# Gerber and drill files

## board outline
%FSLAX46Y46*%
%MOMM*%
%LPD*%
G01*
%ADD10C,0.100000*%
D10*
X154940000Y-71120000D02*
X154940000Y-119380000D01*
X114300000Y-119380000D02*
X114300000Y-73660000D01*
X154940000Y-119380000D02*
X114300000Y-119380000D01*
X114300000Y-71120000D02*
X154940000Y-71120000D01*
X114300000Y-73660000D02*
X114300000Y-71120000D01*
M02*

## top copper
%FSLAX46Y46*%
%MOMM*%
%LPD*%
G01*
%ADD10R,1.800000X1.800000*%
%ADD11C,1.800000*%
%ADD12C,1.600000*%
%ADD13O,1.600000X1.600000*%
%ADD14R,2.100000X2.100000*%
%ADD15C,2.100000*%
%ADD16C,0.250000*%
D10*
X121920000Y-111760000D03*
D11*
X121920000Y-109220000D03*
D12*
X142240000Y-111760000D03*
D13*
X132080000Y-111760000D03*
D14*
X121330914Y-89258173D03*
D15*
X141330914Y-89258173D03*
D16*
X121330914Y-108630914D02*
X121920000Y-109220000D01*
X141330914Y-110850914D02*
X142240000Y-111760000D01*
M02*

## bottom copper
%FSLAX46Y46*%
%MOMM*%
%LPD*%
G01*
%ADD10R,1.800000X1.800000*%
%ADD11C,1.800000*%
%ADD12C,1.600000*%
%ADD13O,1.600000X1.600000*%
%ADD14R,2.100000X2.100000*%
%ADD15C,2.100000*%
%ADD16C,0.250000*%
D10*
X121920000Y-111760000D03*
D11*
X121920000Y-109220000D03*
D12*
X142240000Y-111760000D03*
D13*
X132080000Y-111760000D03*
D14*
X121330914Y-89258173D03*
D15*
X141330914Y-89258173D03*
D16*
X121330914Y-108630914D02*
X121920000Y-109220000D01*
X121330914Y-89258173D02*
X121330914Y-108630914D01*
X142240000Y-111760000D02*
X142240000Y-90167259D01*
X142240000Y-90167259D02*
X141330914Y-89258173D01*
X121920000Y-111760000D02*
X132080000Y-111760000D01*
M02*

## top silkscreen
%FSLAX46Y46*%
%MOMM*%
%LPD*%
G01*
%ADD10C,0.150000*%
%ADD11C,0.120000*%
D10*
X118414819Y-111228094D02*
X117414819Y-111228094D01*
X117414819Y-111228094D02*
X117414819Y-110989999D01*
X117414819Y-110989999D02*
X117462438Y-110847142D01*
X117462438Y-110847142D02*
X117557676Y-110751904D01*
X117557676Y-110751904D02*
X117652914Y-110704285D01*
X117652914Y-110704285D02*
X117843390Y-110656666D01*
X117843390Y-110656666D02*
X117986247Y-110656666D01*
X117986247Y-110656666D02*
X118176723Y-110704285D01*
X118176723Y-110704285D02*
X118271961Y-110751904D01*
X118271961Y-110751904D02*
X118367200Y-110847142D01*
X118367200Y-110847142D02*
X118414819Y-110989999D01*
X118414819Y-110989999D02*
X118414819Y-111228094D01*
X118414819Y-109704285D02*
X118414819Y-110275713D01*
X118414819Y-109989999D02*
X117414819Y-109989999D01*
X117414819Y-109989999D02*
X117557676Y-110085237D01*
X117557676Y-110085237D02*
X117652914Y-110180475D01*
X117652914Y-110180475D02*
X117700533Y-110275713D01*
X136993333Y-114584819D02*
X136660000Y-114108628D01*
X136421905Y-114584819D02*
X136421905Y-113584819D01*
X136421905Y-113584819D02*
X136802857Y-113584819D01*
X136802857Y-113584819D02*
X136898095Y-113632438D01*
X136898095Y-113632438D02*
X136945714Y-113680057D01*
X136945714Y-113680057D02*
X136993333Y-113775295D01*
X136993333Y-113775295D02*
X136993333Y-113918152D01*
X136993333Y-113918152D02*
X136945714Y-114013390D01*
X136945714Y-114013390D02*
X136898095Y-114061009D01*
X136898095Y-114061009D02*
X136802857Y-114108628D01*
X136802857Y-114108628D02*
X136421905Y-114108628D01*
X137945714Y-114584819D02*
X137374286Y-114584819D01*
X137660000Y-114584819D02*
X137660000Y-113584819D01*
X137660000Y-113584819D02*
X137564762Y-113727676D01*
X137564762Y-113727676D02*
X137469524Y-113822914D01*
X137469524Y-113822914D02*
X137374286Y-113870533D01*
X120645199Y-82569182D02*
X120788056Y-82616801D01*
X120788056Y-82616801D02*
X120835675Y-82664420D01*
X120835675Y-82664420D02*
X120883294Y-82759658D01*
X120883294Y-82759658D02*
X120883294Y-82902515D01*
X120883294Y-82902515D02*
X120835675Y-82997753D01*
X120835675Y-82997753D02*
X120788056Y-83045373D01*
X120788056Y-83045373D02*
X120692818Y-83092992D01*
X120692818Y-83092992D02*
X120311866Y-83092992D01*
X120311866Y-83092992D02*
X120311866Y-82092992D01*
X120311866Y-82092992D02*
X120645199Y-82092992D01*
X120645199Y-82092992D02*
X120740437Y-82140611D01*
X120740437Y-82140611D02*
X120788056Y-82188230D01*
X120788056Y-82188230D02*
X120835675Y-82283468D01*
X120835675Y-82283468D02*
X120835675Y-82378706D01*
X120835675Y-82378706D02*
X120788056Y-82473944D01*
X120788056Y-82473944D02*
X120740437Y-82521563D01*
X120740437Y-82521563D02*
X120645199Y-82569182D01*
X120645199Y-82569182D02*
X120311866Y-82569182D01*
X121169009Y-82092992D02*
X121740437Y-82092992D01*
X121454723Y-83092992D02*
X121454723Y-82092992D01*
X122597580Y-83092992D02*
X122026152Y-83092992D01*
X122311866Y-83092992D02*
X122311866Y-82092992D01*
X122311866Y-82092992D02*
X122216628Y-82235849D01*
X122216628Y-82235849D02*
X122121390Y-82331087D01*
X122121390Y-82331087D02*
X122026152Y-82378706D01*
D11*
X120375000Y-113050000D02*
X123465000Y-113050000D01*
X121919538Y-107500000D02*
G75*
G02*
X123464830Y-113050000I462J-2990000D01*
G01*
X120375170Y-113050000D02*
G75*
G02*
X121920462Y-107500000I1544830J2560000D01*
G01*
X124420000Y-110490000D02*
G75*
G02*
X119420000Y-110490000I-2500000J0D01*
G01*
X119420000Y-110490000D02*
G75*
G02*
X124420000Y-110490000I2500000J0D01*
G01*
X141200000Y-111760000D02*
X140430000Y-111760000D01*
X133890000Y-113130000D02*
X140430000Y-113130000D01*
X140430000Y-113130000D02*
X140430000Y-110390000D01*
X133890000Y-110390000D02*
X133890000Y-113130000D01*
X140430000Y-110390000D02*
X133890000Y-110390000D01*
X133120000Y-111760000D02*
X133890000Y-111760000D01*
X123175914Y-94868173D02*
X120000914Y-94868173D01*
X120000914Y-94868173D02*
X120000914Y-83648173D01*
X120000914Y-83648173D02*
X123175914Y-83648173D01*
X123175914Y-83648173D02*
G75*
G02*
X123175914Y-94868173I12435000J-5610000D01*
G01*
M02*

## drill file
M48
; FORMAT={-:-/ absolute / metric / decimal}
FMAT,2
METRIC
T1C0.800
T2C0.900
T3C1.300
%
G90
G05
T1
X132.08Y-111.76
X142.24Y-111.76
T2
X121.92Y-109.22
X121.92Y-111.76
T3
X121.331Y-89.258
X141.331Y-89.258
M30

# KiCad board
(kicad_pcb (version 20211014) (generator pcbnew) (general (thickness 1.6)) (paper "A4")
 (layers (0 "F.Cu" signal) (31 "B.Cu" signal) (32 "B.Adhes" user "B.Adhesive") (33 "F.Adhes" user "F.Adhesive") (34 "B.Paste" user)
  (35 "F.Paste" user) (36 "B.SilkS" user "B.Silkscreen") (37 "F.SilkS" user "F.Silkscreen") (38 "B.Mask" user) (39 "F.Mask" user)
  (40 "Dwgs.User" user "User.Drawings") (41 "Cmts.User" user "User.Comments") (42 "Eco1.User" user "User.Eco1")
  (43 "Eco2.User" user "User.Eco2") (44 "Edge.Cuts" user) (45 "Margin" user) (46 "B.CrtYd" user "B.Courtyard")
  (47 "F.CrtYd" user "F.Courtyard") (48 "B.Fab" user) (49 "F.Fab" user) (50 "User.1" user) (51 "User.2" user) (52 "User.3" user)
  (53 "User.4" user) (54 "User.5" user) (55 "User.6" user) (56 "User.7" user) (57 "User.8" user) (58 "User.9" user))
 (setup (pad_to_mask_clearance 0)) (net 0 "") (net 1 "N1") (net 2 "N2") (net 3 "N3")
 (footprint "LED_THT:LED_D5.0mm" (layer "F.Cu") (at 121.92 111.76 90)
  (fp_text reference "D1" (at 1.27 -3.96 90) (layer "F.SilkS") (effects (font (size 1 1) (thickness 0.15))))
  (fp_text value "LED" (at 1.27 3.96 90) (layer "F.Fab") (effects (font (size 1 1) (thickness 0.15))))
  (fp_line (start -1.29 -1.545) (end -1.29 1.545) (layer "F.SilkS") (width 0.12))
  (fp_arc (start 4.26 -0.000462) (mid 2.072002 2.880433) (end -1.29 1.54483) (layer "F.SilkS") (width 0.12))
  (fp_arc (start -1.29 -1.54483) (mid 2.072002 -2.880433) (end 4.26 0.000462) (layer "F.SilkS") (width 0.12))
  (fp_circle (center 1.27 0) (end 3.77 0) (layer "F.SilkS") (width 0.12) (fill none))
  (pad "1" thru_hole rect (at 0 0 90) (size 1.8 1.8) (drill 0.9) (layers *.Cu *.Mask) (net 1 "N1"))
  (pad "2" thru_hole circle (at 2.54 0 90) (size 1.8 1.8) (drill 0.9) (layers *.Cu *.Mask) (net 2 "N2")))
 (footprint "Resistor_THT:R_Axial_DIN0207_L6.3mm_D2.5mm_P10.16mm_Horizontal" (layer "F.Cu") (at 142.24 111.76 180)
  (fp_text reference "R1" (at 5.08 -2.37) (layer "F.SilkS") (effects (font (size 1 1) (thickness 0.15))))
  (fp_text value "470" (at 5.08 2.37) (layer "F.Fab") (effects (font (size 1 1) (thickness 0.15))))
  (fp_line (start 1.04 0) (end 1.81 0) (layer "F.SilkS") (width 0.12))
  (fp_line (start 8.35 -1.37) (end 1.81 -1.37) (layer "F.SilkS") (width 0.12))
  (fp_line (start 1.81 -1.37) (end 1.81 1.37) (layer "F.SilkS") (width 0.12))
  (fp_line (start 8.35 1.37) (end 8.35 -1.37) (layer "F.SilkS") (width 0.12))
  (fp_line (start 1.81 1.37) (end 8.35 1.37) (layer "F.SilkS") (width 0.12))
  (fp_line (start 9.12 0) (end 8.35 0) (layer "F.SilkS") (width 0.12))
  (pad "1" thru_hole circle (at 0 0 180) (size 1.6 1.6) (drill 0.8) (layers *.Cu *.Mask) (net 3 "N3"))
  (pad "2" thru_hole oval (at 10.16 0 180) (size 1.6 1.6) (drill 0.8) (layers *.Cu *.Mask) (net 1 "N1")))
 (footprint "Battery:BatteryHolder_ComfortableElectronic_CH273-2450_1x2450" (layer "F.Cu") (at 121.330914 89.258173)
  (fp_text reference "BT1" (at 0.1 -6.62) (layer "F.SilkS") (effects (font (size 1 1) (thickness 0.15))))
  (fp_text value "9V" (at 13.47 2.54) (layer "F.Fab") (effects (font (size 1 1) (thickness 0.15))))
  (fp_line (start 1.845 5.61) (end -1.33 5.61) (layer "F.SilkS") (width 0.12))
  (fp_line (start -1.33 5.61) (end -1.33 -5.61) (layer "F.SilkS") (width 0.12))
  (fp_line (start -1.33 -5.61) (end 1.845 -5.61) (layer "F.SilkS") (width 0.12))
  (fp_arc (start 1.845 -5.61) (mid 27.921896 0) (end 1.845 5.61) (layer "F.SilkS") (width 0.12))
  (pad "1" thru_hole rect (at 0 0 270) (size 2.1 2.1) (drill 1.3) (layers *.Cu *.Mask) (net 2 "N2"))
  (pad "2" thru_hole circle (at 20 0 270) (size 2.1 2.1) (drill 1.3) (layers *.Cu *.Mask) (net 3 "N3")))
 (gr_line (start 154.94 71.12) (end 154.94 119.38) (layer "Edge.Cuts") (width 0.1))
 (gr_line (start 114.3 119.38) (end 114.3 73.66) (layer "Edge.Cuts") (width 0.1))
 (gr_line (start 154.94 119.38) (end 114.3 119.38) (layer "Edge.Cuts") (width 0.1))
 (gr_line (start 114.3 71.12) (end 154.94 71.12) (layer "Edge.Cuts") (width 0.1))
 (gr_line (start 114.3 73.66) (end 114.3 71.12) (layer "Edge.Cuts") (width 0.1))
 (segment (start 121.330914 108.630914) (end 121.92 109.22) (width 0.25) (layer "F.Cu") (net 2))
 (segment (start 121.330914 108.630914) (end 121.92 109.22) (width 0.25) (layer "B.Cu") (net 2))
 (segment (start 121.330914 89.258173) (end 121.330914 108.630914) (width 0.25) (layer "B.Cu") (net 2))
 (segment (start 141.330914 110.850914) (end 142.24 111.76) (width 0.25) (layer "F.Cu") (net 3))
 (segment (start 142.24 111.76) (end 142.24 90.167259) (width 0.25) (layer "B.Cu") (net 3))
 (segment (start 142.24 90.167259) (end 141.330914 89.258173) (width 0.25) (layer "B.Cu") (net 3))
 (segment (start 121.92 111.76) (end 132.08 111.76) (width 0.25) (layer "B.Cu") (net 1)))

